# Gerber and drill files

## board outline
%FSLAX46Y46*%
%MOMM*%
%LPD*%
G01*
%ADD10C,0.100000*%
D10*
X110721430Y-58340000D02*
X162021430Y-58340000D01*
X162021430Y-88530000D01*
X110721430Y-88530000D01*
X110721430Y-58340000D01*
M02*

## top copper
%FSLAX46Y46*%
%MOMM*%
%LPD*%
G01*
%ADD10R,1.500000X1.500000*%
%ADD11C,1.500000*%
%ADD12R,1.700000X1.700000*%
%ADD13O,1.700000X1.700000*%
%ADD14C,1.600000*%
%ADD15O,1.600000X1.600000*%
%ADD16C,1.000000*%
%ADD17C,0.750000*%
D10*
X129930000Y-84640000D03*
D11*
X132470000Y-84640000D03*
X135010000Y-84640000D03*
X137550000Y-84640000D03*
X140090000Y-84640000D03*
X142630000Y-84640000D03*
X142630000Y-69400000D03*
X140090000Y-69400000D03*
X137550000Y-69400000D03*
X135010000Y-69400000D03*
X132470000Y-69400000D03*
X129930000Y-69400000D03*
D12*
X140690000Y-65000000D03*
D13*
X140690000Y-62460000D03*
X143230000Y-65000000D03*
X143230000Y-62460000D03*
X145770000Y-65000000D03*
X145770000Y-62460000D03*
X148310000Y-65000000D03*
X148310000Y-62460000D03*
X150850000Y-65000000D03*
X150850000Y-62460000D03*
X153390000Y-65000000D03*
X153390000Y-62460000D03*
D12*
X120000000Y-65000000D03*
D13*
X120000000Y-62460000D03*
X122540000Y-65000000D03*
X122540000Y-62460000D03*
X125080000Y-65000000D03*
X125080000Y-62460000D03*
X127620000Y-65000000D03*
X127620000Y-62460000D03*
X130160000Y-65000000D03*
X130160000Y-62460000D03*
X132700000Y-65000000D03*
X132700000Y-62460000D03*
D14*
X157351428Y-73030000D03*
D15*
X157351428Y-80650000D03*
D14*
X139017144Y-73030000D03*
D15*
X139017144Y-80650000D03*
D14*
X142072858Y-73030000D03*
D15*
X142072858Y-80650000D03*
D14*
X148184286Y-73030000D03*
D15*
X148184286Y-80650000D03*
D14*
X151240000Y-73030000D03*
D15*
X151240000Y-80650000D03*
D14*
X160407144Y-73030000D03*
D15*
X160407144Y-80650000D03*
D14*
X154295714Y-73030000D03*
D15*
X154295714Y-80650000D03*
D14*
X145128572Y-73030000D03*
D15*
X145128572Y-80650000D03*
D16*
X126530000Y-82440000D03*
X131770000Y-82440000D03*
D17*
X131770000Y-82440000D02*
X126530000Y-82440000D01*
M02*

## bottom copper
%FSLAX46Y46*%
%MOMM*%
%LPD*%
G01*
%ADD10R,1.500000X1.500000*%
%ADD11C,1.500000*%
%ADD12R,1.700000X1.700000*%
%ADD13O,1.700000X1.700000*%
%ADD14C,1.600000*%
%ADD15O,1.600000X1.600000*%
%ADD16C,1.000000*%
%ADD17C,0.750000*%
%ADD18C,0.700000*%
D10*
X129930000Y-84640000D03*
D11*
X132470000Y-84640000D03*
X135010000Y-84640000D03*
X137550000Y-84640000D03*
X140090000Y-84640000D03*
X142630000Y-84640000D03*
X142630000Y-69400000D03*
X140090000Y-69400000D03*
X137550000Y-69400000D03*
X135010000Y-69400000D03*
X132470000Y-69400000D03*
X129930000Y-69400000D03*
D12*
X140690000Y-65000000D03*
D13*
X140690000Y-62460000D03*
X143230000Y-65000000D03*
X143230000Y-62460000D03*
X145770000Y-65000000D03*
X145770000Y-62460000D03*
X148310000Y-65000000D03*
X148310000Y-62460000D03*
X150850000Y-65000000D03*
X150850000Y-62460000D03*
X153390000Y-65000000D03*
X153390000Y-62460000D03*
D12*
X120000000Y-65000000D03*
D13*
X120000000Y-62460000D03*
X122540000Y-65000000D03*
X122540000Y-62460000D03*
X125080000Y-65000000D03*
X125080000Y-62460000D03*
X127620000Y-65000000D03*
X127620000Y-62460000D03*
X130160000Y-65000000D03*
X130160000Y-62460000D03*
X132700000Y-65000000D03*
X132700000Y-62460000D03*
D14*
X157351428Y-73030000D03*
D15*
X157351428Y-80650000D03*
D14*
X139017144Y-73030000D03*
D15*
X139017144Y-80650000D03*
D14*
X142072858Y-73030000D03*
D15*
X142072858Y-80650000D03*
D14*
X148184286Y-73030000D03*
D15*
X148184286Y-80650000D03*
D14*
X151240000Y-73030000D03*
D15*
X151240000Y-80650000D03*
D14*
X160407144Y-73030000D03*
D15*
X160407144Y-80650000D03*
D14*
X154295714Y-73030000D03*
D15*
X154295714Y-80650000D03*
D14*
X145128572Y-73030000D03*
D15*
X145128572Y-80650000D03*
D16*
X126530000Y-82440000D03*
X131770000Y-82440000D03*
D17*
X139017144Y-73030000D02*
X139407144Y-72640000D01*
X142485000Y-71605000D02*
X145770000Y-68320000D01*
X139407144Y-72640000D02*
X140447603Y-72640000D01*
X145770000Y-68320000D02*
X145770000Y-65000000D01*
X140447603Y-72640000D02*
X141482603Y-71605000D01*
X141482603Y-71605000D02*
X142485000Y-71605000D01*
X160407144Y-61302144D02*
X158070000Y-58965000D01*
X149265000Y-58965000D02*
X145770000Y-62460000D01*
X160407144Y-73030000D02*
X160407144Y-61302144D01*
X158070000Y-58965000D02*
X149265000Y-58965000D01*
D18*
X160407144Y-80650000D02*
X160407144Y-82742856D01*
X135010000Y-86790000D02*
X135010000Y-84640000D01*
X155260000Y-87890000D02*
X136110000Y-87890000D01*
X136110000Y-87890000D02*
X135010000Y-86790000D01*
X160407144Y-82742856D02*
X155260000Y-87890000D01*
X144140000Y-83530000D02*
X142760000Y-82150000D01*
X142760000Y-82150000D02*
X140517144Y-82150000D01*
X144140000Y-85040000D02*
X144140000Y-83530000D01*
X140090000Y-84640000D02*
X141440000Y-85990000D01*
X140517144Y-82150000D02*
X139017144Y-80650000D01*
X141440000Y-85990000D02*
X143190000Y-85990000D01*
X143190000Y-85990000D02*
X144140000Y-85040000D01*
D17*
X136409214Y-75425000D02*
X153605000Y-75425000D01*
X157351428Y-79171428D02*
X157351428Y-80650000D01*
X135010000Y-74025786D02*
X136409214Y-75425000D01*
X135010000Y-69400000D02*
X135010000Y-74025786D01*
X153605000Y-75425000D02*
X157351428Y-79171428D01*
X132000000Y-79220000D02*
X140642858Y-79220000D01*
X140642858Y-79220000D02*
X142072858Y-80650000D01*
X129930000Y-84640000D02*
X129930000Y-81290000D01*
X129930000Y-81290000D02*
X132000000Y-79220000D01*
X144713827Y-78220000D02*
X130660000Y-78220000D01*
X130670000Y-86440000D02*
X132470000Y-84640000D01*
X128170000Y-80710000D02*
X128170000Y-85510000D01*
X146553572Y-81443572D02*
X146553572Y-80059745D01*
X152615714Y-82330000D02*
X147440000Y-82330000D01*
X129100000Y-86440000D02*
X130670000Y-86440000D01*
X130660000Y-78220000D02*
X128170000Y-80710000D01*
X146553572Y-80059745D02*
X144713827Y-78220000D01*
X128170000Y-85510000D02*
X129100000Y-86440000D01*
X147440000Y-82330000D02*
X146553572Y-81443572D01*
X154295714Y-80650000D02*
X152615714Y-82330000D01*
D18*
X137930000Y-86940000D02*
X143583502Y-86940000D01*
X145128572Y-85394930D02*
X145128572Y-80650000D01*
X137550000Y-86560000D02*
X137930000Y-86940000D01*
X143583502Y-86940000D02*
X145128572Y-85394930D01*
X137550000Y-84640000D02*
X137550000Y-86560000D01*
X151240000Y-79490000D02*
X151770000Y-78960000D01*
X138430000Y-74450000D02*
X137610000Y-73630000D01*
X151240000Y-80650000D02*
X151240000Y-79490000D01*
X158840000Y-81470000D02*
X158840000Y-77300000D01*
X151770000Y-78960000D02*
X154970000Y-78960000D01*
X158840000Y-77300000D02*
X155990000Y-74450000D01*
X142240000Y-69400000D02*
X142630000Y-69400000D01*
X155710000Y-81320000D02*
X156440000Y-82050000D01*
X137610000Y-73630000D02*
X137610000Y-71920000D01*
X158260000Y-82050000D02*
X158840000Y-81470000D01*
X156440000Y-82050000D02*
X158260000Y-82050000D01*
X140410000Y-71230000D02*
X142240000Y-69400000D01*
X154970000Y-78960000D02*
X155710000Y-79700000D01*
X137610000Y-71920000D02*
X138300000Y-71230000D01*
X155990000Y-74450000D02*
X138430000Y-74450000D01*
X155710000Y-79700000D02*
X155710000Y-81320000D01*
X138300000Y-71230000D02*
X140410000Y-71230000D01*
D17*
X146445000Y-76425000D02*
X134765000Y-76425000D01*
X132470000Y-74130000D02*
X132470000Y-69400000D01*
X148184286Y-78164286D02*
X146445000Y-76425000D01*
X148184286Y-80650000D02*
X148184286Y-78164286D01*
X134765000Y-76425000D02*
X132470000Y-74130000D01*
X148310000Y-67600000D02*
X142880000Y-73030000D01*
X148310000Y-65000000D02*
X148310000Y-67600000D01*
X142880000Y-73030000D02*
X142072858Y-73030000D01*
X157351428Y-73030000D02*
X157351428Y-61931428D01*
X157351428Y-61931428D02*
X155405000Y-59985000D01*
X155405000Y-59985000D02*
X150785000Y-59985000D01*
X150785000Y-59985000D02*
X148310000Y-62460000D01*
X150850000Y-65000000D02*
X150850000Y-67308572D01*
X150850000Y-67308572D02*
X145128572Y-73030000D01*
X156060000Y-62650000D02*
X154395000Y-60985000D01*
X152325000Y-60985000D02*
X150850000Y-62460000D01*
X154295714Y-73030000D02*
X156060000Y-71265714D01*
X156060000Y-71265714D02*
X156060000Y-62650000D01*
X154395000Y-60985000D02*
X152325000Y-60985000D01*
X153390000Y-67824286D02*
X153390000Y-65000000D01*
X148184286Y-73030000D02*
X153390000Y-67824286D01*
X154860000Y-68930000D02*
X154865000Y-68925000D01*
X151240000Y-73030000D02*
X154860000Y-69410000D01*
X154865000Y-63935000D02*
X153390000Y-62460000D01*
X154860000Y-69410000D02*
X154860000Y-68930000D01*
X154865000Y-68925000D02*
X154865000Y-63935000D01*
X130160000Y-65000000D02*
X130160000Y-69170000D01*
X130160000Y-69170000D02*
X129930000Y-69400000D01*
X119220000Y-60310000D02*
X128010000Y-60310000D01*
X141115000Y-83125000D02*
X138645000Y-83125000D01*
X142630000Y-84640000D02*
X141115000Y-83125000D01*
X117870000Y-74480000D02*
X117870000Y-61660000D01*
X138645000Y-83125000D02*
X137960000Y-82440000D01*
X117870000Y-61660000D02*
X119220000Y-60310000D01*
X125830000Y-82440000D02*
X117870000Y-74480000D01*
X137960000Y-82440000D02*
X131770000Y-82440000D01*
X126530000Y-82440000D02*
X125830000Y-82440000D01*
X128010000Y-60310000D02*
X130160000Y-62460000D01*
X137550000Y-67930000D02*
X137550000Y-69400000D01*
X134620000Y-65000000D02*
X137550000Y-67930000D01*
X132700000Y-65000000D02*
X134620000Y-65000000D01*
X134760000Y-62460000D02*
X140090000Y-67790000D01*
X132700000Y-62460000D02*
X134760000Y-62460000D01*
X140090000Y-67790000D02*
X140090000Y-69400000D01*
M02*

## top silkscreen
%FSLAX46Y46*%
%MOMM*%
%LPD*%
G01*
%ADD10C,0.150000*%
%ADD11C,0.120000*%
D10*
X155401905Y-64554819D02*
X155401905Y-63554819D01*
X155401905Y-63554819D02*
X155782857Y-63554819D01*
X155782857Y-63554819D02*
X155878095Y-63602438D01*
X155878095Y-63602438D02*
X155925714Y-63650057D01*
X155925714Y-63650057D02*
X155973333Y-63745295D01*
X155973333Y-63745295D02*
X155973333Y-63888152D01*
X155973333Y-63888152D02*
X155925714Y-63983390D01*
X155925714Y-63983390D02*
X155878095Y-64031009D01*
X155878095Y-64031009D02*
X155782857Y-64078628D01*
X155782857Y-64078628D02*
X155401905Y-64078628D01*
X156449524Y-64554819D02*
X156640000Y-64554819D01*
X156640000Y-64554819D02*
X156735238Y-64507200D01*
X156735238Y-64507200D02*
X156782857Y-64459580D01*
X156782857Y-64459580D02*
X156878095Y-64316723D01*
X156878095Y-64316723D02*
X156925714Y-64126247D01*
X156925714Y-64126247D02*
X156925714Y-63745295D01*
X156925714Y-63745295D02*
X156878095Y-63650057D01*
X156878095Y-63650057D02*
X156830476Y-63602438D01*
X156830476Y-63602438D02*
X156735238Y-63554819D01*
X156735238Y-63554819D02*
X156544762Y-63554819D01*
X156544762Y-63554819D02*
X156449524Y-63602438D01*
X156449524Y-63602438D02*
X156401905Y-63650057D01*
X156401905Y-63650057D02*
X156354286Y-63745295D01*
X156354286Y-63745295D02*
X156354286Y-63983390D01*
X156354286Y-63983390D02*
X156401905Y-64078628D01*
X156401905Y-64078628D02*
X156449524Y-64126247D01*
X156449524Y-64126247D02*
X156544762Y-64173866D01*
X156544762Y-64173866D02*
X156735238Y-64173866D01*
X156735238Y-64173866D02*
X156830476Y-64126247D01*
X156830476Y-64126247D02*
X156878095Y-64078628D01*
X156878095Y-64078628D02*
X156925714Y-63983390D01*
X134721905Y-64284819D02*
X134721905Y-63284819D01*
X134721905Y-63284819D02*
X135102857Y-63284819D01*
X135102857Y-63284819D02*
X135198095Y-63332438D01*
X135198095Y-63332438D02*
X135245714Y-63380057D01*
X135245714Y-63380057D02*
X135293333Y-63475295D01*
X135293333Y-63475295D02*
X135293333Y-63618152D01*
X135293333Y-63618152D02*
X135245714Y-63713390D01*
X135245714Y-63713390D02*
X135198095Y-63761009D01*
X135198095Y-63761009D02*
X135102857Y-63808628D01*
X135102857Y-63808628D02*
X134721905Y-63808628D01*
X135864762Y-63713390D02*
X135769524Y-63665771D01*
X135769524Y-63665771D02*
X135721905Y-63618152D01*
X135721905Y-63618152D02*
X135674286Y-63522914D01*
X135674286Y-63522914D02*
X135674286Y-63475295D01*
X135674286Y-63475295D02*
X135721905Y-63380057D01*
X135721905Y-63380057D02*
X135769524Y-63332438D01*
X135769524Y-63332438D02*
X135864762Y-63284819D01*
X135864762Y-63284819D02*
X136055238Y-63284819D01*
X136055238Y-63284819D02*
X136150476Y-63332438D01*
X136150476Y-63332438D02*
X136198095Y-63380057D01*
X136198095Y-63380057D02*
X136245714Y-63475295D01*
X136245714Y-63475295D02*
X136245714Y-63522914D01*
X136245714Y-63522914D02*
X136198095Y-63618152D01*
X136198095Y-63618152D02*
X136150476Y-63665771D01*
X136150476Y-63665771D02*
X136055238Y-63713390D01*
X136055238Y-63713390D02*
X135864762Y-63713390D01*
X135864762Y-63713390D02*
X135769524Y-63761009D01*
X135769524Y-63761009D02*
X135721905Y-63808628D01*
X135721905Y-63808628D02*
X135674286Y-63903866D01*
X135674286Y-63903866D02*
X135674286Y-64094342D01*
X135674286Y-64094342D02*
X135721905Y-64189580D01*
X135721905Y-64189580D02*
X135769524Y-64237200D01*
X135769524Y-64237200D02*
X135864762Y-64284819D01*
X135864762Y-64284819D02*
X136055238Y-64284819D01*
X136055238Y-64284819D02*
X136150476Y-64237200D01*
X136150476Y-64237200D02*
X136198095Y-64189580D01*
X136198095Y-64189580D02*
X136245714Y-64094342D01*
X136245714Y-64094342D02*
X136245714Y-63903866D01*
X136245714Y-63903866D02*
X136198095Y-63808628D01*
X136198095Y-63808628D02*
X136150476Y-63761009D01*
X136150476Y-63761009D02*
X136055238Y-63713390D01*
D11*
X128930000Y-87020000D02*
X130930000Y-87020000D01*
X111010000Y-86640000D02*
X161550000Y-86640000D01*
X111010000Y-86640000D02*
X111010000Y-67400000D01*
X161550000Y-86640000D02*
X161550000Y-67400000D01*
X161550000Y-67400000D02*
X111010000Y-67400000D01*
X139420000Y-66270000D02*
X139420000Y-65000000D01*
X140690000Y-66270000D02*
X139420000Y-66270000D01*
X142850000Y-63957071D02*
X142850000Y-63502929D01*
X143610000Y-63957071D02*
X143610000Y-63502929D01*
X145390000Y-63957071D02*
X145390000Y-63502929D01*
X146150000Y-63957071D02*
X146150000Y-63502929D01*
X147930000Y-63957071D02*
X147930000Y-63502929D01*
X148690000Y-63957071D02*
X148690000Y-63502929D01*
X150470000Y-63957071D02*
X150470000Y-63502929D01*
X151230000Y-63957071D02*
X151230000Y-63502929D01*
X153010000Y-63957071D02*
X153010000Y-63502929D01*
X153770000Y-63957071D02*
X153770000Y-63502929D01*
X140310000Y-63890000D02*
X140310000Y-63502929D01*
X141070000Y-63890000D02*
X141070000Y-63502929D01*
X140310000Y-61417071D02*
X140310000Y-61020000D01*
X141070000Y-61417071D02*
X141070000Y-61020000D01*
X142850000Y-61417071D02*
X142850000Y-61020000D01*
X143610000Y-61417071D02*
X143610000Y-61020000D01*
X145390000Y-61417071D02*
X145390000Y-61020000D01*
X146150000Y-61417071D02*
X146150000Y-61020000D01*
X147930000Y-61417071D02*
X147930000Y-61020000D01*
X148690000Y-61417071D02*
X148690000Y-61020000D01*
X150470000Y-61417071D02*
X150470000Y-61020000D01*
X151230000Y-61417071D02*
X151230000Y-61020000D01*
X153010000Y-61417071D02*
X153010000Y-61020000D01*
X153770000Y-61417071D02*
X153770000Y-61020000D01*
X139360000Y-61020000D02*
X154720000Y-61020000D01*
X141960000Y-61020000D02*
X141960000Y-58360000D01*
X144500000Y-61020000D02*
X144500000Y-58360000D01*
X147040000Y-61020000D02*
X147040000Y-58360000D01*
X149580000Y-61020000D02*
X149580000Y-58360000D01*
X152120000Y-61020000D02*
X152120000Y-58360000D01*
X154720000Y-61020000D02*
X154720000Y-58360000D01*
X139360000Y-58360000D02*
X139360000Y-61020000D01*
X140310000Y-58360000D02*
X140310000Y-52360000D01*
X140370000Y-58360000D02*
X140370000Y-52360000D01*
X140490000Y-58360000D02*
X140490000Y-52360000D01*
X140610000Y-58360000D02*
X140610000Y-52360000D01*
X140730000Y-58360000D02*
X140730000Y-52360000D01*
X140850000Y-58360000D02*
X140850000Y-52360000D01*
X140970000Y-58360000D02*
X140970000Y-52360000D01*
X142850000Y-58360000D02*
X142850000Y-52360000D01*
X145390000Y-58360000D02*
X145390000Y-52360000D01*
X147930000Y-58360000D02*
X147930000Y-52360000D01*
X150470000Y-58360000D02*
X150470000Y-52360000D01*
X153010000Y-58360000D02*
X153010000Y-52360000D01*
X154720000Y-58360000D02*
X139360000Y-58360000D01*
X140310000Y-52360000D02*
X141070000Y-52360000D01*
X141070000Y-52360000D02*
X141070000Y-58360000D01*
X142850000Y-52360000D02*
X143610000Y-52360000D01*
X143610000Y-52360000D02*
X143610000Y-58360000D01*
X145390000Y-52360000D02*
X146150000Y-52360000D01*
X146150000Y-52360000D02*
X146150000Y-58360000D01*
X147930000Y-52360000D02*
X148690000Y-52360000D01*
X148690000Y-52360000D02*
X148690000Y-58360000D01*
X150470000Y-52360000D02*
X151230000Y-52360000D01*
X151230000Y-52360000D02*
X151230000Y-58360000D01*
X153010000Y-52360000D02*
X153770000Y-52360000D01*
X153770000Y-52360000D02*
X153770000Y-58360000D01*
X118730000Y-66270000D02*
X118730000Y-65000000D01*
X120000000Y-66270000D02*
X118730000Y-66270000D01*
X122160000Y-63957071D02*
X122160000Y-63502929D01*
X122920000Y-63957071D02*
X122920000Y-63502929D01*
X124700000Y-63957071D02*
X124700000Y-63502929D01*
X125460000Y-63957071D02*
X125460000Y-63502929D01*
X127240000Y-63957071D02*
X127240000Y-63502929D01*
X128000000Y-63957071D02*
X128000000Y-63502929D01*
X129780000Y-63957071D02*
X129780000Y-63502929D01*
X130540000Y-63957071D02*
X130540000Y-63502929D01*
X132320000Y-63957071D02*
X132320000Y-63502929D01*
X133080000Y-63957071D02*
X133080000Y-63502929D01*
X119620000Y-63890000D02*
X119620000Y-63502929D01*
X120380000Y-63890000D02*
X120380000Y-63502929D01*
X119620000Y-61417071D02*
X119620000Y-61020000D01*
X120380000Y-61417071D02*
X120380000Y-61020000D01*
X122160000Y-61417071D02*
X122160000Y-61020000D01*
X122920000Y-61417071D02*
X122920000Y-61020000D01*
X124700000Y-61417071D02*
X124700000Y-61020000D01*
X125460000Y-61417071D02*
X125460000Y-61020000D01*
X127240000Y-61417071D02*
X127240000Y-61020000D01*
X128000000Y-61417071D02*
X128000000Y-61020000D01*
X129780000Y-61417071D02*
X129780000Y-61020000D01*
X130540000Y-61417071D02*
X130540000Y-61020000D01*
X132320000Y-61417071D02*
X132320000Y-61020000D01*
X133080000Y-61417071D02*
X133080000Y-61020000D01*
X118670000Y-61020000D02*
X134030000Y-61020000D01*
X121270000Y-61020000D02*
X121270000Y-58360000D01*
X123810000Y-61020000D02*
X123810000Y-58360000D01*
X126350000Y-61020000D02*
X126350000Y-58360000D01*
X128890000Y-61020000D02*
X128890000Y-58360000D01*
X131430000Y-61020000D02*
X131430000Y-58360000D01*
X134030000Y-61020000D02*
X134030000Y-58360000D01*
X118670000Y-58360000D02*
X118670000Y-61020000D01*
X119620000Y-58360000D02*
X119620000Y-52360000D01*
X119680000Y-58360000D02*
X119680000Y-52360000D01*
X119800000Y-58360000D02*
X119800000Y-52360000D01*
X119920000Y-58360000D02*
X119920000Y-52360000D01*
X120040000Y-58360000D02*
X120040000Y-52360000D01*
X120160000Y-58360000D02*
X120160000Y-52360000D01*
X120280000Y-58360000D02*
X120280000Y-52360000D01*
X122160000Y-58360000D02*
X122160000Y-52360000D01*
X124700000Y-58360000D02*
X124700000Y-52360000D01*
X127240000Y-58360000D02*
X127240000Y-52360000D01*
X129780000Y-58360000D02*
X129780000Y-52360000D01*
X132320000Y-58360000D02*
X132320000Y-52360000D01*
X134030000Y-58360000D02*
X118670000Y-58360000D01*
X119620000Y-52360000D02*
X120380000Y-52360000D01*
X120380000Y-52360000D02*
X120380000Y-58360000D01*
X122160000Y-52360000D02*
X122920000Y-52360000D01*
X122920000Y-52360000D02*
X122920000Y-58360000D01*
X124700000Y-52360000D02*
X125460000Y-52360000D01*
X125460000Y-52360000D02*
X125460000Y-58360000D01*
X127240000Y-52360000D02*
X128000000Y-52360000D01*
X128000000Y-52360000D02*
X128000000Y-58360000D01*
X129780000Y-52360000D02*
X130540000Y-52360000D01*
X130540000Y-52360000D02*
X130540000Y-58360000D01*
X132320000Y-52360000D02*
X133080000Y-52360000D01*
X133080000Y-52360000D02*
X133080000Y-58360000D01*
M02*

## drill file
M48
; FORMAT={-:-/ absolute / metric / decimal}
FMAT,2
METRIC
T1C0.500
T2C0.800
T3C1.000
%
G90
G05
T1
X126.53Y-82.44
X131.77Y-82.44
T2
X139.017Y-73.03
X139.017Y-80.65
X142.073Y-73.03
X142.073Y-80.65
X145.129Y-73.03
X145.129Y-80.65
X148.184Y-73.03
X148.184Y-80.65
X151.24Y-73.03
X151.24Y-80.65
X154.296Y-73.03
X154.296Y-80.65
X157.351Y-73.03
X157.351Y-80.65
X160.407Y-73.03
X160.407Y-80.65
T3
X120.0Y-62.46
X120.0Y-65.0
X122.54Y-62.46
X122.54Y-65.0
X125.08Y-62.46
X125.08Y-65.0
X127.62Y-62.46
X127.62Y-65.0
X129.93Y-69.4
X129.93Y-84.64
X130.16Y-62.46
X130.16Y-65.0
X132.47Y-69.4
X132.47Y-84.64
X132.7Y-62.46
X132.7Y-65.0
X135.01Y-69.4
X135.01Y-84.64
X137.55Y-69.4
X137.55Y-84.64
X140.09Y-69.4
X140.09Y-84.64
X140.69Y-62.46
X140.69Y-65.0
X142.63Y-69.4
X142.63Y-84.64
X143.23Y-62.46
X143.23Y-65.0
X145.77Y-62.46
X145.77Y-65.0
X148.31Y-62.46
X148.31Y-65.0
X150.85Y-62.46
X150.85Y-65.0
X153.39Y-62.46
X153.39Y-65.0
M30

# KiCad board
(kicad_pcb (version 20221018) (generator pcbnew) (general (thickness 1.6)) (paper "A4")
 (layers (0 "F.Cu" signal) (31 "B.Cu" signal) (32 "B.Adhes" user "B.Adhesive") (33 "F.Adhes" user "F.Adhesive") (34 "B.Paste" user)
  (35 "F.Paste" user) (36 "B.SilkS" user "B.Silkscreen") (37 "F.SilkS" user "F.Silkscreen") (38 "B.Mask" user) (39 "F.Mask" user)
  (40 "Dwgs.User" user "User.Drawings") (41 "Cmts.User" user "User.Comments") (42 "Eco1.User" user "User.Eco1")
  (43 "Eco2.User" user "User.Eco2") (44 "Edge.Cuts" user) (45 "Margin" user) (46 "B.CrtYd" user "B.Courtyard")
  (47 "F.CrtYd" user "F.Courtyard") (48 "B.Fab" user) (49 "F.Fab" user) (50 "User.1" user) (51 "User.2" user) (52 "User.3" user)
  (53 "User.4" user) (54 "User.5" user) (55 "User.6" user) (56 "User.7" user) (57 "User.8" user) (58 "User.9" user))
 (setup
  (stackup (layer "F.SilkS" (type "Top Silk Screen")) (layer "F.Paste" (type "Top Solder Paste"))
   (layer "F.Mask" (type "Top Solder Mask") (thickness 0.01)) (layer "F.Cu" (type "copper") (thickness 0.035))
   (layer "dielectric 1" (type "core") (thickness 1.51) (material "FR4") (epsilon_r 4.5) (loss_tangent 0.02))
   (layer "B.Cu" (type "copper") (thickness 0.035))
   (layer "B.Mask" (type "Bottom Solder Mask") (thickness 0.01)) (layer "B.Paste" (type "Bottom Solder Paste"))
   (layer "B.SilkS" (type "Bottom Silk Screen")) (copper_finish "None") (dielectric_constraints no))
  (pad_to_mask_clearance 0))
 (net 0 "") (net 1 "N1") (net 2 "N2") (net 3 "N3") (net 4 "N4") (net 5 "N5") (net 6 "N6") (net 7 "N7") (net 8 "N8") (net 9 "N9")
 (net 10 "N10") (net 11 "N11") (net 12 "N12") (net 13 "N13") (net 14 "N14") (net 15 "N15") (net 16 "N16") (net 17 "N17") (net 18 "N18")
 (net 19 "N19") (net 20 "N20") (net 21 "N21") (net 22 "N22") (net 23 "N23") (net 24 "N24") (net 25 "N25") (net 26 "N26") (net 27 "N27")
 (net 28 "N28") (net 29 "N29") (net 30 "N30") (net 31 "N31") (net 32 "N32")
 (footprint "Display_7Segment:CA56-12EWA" (layer "F.Cu") (at 129.93 84.64 90)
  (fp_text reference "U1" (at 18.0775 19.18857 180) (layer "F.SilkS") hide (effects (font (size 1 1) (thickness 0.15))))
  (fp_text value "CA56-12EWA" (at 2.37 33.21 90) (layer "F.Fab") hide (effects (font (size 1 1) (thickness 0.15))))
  (fp_line (start -2.38 -1) (end -2.38 1) (stroke (width 0.12) (type solid)) (layer "F.SilkS"))
  (fp_line (start -2 -18.92) (end -2 31.62) (stroke (width 0.12) (type solid)) (layer "F.SilkS"))
  (fp_line (start -2 -18.92) (end 17.24 -18.92) (stroke (width 0.12) (type solid)) (layer "F.SilkS"))
  (fp_line (start -2 31.62) (end 17.24 31.62) (stroke (width 0.12) (type solid)) (layer "F.SilkS"))
  (fp_line (start 17.24 31.62) (end 17.24 -18.92) (stroke (width 0.12) (type solid)) (layer "F.SilkS"))
  (pad "1" thru_hole rect (at 0 0 90) (size 1.5 1.5) (drill 1) (layers "*.Cu" "*.Mask") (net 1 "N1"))
  (pad "2" thru_hole circle (at 0 2.54 90) (size 1.5 1.5) (drill 1) (layers "*.Cu" "*.Mask") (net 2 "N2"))
  (pad "3" thru_hole circle (at 0 5.08 90) (size 1.5 1.5) (drill 1) (layers "*.Cu" "*.Mask") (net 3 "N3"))
  (pad "4" thru_hole circle (at 0 7.62 90) (size 1.5 1.5) (drill 1) (layers "*.Cu" "*.Mask") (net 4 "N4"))
  (pad "5" thru_hole circle (at 0 10.16 90) (size 1.5 1.5) (drill 1) (layers "*.Cu" "*.Mask") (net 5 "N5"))
  (pad "6" thru_hole circle (at 0 12.7 90) (size 1.5 1.5) (drill 1) (layers "*.Cu" "*.Mask") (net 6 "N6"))
  (pad "7" thru_hole circle (at 15.24 12.7 90) (size 1.5 1.5) (drill 1) (layers "*.Cu" "*.Mask") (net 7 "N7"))
  (pad "8" thru_hole circle (at 15.24 10.16 90) (size 1.5 1.5) (drill 1) (layers "*.Cu" "*.Mask") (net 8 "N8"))
  (pad "9" thru_hole circle (at 15.24 7.62 90) (size 1.5 1.5) (drill 1) (layers "*.Cu" "*.Mask") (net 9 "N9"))
  (pad "10" thru_hole circle (at 15.24 5.08 90) (size 1.5 1.5) (drill 1) (layers "*.Cu" "*.Mask") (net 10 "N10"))
  (pad "11" thru_hole circle (at 15.24 2.54 90) (size 1.5 1.5) (drill 1) (layers "*.Cu" "*.Mask") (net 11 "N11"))
  (pad "12" thru_hole circle (at 15.24 0 90) (size 1.5 1.5) (drill 1) (layers "*.Cu" "*.Mask") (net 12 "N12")))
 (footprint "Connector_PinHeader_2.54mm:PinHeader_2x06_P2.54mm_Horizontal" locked (layer "F.Cu") (at 140.69 65 90)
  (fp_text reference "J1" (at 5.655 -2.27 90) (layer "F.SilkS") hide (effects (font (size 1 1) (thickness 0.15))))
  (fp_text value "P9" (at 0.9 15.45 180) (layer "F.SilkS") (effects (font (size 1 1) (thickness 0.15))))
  (fp_line (start -1.27 -1.27) (end 0 -1.27) (stroke (width 0.12) (type solid)) (layer "F.SilkS"))
  (fp_line (start -1.27 0) (end -1.27 -1.27) (stroke (width 0.12) (type solid)) (layer "F.SilkS"))
  (fp_line (start 1.042929 2.16) (end 1.497071 2.16) (stroke (width 0.12) (type solid)) (layer "F.SilkS"))
  (fp_line (start 1.042929 2.92) (end 1.497071 2.92) (stroke (width 0.12) (type solid)) (layer "F.SilkS"))
  (fp_line (start 1.042929 4.7) (end 1.497071 4.7) (stroke (width 0.12) (type solid)) (layer "F.SilkS"))
  (fp_line (start 1.042929 5.46) (end 1.497071 5.46) (stroke (width 0.12) (type solid)) (layer "F.SilkS"))
  (fp_line (start 1.042929 7.24) (end 1.497071 7.24) (stroke (width 0.12) (type solid)) (layer "F.SilkS"))
  (fp_line (start 1.042929 8) (end 1.497071 8) (stroke (width 0.12) (type solid)) (layer "F.SilkS"))
  (fp_line (start 1.042929 9.78) (end 1.497071 9.78) (stroke (width 0.12) (type solid)) (layer "F.SilkS"))
  (fp_line (start 1.042929 10.54) (end 1.497071 10.54) (stroke (width 0.12) (type solid)) (layer "F.SilkS"))
  (fp_line (start 1.042929 12.32) (end 1.497071 12.32) (stroke (width 0.12) (type solid)) (layer "F.SilkS"))
  (fp_line (start 1.042929 13.08) (end 1.497071 13.08) (stroke (width 0.12) (type solid)) (layer "F.SilkS"))
  (fp_line (start 1.11 -0.38) (end 1.497071 -0.38) (stroke (width 0.12) (type solid)) (layer "F.SilkS"))
  (fp_line (start 1.11 0.38) (end 1.497071 0.38) (stroke (width 0.12) (type solid)) (layer "F.SilkS"))
  (fp_line (start 3.582929 -0.38) (end 3.98 -0.38) (stroke (width 0.12) (type solid)) (layer "F.SilkS"))
  (fp_line (start 3.582929 0.38) (end 3.98 0.38) (stroke (width 0.12) (type solid)) (layer "F.SilkS"))
  (fp_line (start 3.582929 2.16) (end 3.98 2.16) (stroke (width 0.12) (type solid)) (layer "F.SilkS"))
  (fp_line (start 3.582929 2.92) (end 3.98 2.92) (stroke (width 0.12) (type solid)) (layer "F.SilkS"))
  (fp_line (start 3.582929 4.7) (end 3.98 4.7) (stroke (width 0.12) (type solid)) (layer "F.SilkS"))
  (fp_line (start 3.582929 5.46) (end 3.98 5.46) (stroke (width 0.12) (type solid)) (layer "F.SilkS"))
  (fp_line (start 3.582929 7.24) (end 3.98 7.24) (stroke (width 0.12) (type solid)) (layer "F.SilkS"))
  (fp_line (start 3.582929 8) (end 3.98 8) (stroke (width 0.12) (type solid)) (layer "F.SilkS"))
  (fp_line (start 3.582929 9.78) (end 3.98 9.78) (stroke (width 0.12) (type solid)) (layer "F.SilkS"))
  (fp_line (start 3.582929 10.54) (end 3.98 10.54) (stroke (width 0.12) (type solid)) (layer "F.SilkS"))
  (fp_line (start 3.582929 12.32) (end 3.98 12.32) (stroke (width 0.12) (type solid)) (layer "F.SilkS"))
  (fp_line (start 3.582929 13.08) (end 3.98 13.08) (stroke (width 0.12) (type solid)) (layer "F.SilkS"))
  (fp_line (start 3.98 -1.33) (end 3.98 14.03) (stroke (width 0.12) (type solid)) (layer "F.SilkS"))
  (fp_line (start 3.98 1.27) (end 6.64 1.27) (stroke (width 0.12) (type solid)) (layer "F.SilkS"))
  (fp_line (start 3.98 3.81) (end 6.64 3.81) (stroke (width 0.12) (type solid)) (layer "F.SilkS"))
  (fp_line (start 3.98 6.35) (end 6.64 6.35) (stroke (width 0.12) (type solid)) (layer "F.SilkS"))
  (fp_line (start 3.98 8.89) (end 6.64 8.89) (stroke (width 0.12) (type solid)) (layer "F.SilkS"))
  (fp_line (start 3.98 11.43) (end 6.64 11.43) (stroke (width 0.12) (type solid)) (layer "F.SilkS"))
  (fp_line (start 3.98 14.03) (end 6.64 14.03) (stroke (width 0.12) (type solid)) (layer "F.SilkS"))
  (fp_line (start 6.64 -1.33) (end 3.98 -1.33) (stroke (width 0.12) (type solid)) (layer "F.SilkS"))
  (fp_line (start 6.64 -0.38) (end 12.64 -0.38) (stroke (width 0.12) (type solid)) (layer "F.SilkS"))
  (fp_line (start 6.64 -0.32) (end 12.64 -0.32) (stroke (width 0.12) (type solid)) (layer "F.SilkS"))
  (fp_line (start 6.64 -0.2) (end 12.64 -0.2) (stroke (width 0.12) (type solid)) (layer "F.SilkS"))
  (fp_line (start 6.64 -0.08) (end 12.64 -0.08) (stroke (width 0.12) (type solid)) (layer "F.SilkS"))
  (fp_line (start 6.64 0.04) (end 12.64 0.04) (stroke (width 0.12) (type solid)) (layer "F.SilkS"))
  (fp_line (start 6.64 0.16) (end 12.64 0.16) (stroke (width 0.12) (type solid)) (layer "F.SilkS"))
  (fp_line (start 6.64 0.28) (end 12.64 0.28) (stroke (width 0.12) (type solid)) (layer "F.SilkS"))
  (fp_line (start 6.64 2.16) (end 12.64 2.16) (stroke (width 0.12) (type solid)) (layer "F.SilkS"))
  (fp_line (start 6.64 4.7) (end 12.64 4.7) (stroke (width 0.12) (type solid)) (layer "F.SilkS"))
  (fp_line (start 6.64 7.24) (end 12.64 7.24) (stroke (width 0.12) (type solid)) (layer "F.SilkS"))
  (fp_line (start 6.64 9.78) (end 12.64 9.78) (stroke (width 0.12) (type solid)) (layer "F.SilkS"))
  (fp_line (start 6.64 12.32) (end 12.64 12.32) (stroke (width 0.12) (type solid)) (layer "F.SilkS"))
  (fp_line (start 6.64 14.03) (end 6.64 -1.33) (stroke (width 0.12) (type solid)) (layer "F.SilkS"))
  (fp_line (start 12.64 -0.38) (end 12.64 0.38) (stroke (width 0.12) (type solid)) (layer "F.SilkS"))
  (fp_line (start 12.64 0.38) (end 6.64 0.38) (stroke (width 0.12) (type solid)) (layer "F.SilkS"))
  (fp_line (start 12.64 2.16) (end 12.64 2.92) (stroke (width 0.12) (type solid)) (layer "F.SilkS"))
  (fp_line (start 12.64 2.92) (end 6.64 2.92) (stroke (width 0.12) (type solid)) (layer "F.SilkS"))
  (fp_line (start 12.64 4.7) (end 12.64 5.46) (stroke (width 0.12) (type solid)) (layer "F.SilkS"))
  (fp_line (start 12.64 5.46) (end 6.64 5.46) (stroke (width 0.12) (type solid)) (layer "F.SilkS"))
  (fp_line (start 12.64 7.24) (end 12.64 8) (stroke (width 0.12) (type solid)) (layer "F.SilkS"))
  (fp_line (start 12.64 8) (end 6.64 8) (stroke (width 0.12) (type solid)) (layer "F.SilkS"))
  (fp_line (start 12.64 9.78) (end 12.64 10.54) (stroke (width 0.12) (type solid)) (layer "F.SilkS"))
  (fp_line (start 12.64 10.54) (end 6.64 10.54) (stroke (width 0.12) (type solid)) (layer "F.SilkS"))
  (fp_line (start 12.64 12.32) (end 12.64 13.08) (stroke (width 0.12) (type solid)) (layer "F.SilkS"))
  (fp_line (start 12.64 13.08) (end 6.64 13.08) (stroke (width 0.12) (type solid)) (layer "F.SilkS"))
  (pad "1" thru_hole rect locked (at 0 0 90) (size 1.7 1.7) (drill 1) (layers "*.Cu" "*.Mask") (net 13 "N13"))
  (pad "2" thru_hole oval locked (at 2.54 0 90) (size 1.7 1.7) (drill 1) (layers "*.Cu" "*.Mask") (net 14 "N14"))
  (pad "3" thru_hole oval locked (at 0 2.54 90) (size 1.7 1.7) (drill 1) (layers "*.Cu" "*.Mask") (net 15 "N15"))
  (pad "4" thru_hole oval locked (at 2.54 2.54 90) (size 1.7 1.7) (drill 1) (layers "*.Cu" "*.Mask") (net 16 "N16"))
  (pad "5" thru_hole oval locked (at 0 5.08 90) (size 1.7 1.7) (drill 1) (layers "*.Cu" "*.Mask") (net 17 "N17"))
  (pad "6" thru_hole oval locked (at 2.54 5.08 90) (size 1.7 1.7) (drill 1) (layers "*.Cu" "*.Mask") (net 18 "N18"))
  (pad "7" thru_hole oval locked (at 0 7.62 90) (size 1.7 1.7) (drill 1) (layers "*.Cu" "*.Mask") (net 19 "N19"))
  (pad "8" thru_hole oval locked (at 2.54 7.62 90) (size 1.7 1.7) (drill 1) (layers "*.Cu" "*.Mask") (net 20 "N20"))
  (pad "9" thru_hole oval locked (at 0 10.16 90) (size 1.7 1.7) (drill 1) (layers "*.Cu" "*.Mask") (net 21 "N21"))
  (pad "10" thru_hole oval locked (at 2.54 10.16 90) (size 1.7 1.7) (drill 1) (layers "*.Cu" "*.Mask") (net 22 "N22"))
  (pad "11" thru_hole oval locked (at 0 12.7 90) (size 1.7 1.7) (drill 1) (layers "*.Cu" "*.Mask") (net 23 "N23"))
  (pad "12" thru_hole oval locked (at 2.54 12.7 90) (size 1.7 1.7) (drill 1) (layers "*.Cu" "*.Mask") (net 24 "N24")))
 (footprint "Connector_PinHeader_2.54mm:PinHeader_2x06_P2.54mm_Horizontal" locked (layer "F.Cu") (at 120 65 90)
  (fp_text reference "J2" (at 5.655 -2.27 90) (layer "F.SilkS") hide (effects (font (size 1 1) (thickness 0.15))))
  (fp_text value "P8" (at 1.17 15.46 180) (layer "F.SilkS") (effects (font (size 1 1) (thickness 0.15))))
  (fp_line (start -1.27 -1.27) (end 0 -1.27) (stroke (width 0.12) (type solid)) (layer "F.SilkS"))
  (fp_line (start -1.27 0) (end -1.27 -1.27) (stroke (width 0.12) (type solid)) (layer "F.SilkS"))
  (fp_line (start 1.042929 2.16) (end 1.497071 2.16) (stroke (width 0.12) (type solid)) (layer "F.SilkS"))
  (fp_line (start 1.042929 2.92) (end 1.497071 2.92) (stroke (width 0.12) (type solid)) (layer "F.SilkS"))
  (fp_line (start 1.042929 4.7) (end 1.497071 4.7) (stroke (width 0.12) (type solid)) (layer "F.SilkS"))
  (fp_line (start 1.042929 5.46) (end 1.497071 5.46) (stroke (width 0.12) (type solid)) (layer "F.SilkS"))
  (fp_line (start 1.042929 7.24) (end 1.497071 7.24) (stroke (width 0.12) (type solid)) (layer "F.SilkS"))
  (fp_line (start 1.042929 8) (end 1.497071 8) (stroke (width 0.12) (type solid)) (layer "F.SilkS"))
  (fp_line (start 1.042929 9.78) (end 1.497071 9.78) (stroke (width 0.12) (type solid)) (layer "F.SilkS"))
  (fp_line (start 1.042929 10.54) (end 1.497071 10.54) (stroke (width 0.12) (type solid)) (layer "F.SilkS"))
  (fp_line (start 1.042929 12.32) (end 1.497071 12.32) (stroke (width 0.12) (type solid)) (layer "F.SilkS"))
  (fp_line (start 1.042929 13.08) (end 1.497071 13.08) (stroke (width 0.12) (type solid)) (layer "F.SilkS"))
  (fp_line (start 1.11 -0.38) (end 1.497071 -0.38) (stroke (width 0.12) (type solid)) (layer "F.SilkS"))
  (fp_line (start 1.11 0.38) (end 1.497071 0.38) (stroke (width 0.12) (type solid)) (layer "F.SilkS"))
  (fp_line (start 3.582929 -0.38) (end 3.98 -0.38) (stroke (width 0.12) (type solid)) (layer "F.SilkS"))
  (fp_line (start 3.582929 0.38) (end 3.98 0.38) (stroke (width 0.12) (type solid)) (layer "F.SilkS"))
  (fp_line (start 3.582929 2.16) (end 3.98 2.16) (stroke (width 0.12) (type solid)) (layer "F.SilkS"))
  (fp_line (start 3.582929 2.92) (end 3.98 2.92) (stroke (width 0.12) (type solid)) (layer "F.SilkS"))
  (fp_line (start 3.582929 4.7) (end 3.98 4.7) (stroke (width 0.12) (type solid)) (layer "F.SilkS"))
  (fp_line (start 3.582929 5.46) (end 3.98 5.46) (stroke (width 0.12) (type solid)) (layer "F.SilkS"))
  (fp_line (start 3.582929 7.24) (end 3.98 7.24) (stroke (width 0.12) (type solid)) (layer "F.SilkS"))
  (fp_line (start 3.582929 8) (end 3.98 8) (stroke (width 0.12) (type solid)) (layer "F.SilkS"))
  (fp_line (start 3.582929 9.78) (end 3.98 9.78) (stroke (width 0.12) (type solid)) (layer "F.SilkS"))
  (fp_line (start 3.582929 10.54) (end 3.98 10.54) (stroke (width 0.12) (type solid)) (layer "F.SilkS"))
  (fp_line (start 3.582929 12.32) (end 3.98 12.32) (stroke (width 0.12) (type solid)) (layer "F.SilkS"))
  (fp_line (start 3.582929 13.08) (end 3.98 13.08) (stroke (width 0.12) (type solid)) (layer "F.SilkS"))
  (fp_line (start 3.98 -1.33) (end 3.98 14.03) (stroke (width 0.12) (type solid)) (layer "F.SilkS"))
  (fp_line (start 3.98 1.27) (end 6.64 1.27) (stroke (width 0.12) (type solid)) (layer "F.SilkS"))
  (fp_line (start 3.98 3.81) (end 6.64 3.81) (stroke (width 0.12) (type solid)) (layer "F.SilkS"))
  (fp_line (start 3.98 6.35) (end 6.64 6.35) (stroke (width 0.12) (type solid)) (layer "F.SilkS"))
  (fp_line (start 3.98 8.89) (end 6.64 8.89) (stroke (width 0.12) (type solid)) (layer "F.SilkS"))
  (fp_line (start 3.98 11.43) (end 6.64 11.43) (stroke (width 0.12) (type solid)) (layer "F.SilkS"))
  (fp_line (start 3.98 14.03) (end 6.64 14.03) (stroke (width 0.12) (type solid)) (layer "F.SilkS"))
  (fp_line (start 6.64 -1.33) (end 3.98 -1.33) (stroke (width 0.12) (type solid)) (layer "F.SilkS"))
  (fp_line (start 6.64 -0.38) (end 12.64 -0.38) (stroke (width 0.12) (type solid)) (layer "F.SilkS"))
  (fp_line (start 6.64 -0.32) (end 12.64 -0.32) (stroke (width 0.12) (type solid)) (layer "F.SilkS"))
  (fp_line (start 6.64 -0.2) (end 12.64 -0.2) (stroke (width 0.12) (type solid)) (layer "F.SilkS"))
  (fp_line (start 6.64 -0.08) (end 12.64 -0.08) (stroke (width 0.12) (type solid)) (layer "F.SilkS"))
  (fp_line (start 6.64 0.04) (end 12.64 0.04) (stroke (width 0.12) (type solid)) (layer "F.SilkS"))
  (fp_line (start 6.64 0.16) (end 12.64 0.16) (stroke (width 0.12) (type solid)) (layer "F.SilkS"))
  (fp_line (start 6.64 0.28) (end 12.64 0.28) (stroke (width 0.12) (type solid)) (layer "F.SilkS"))
  (fp_line (start 6.64 2.16) (end 12.64 2.16) (stroke (width 0.12) (type solid)) (layer "F.SilkS"))
  (fp_line (start 6.64 4.7) (end 12.64 4.7) (stroke (width 0.12) (type solid)) (layer "F.SilkS"))
  (fp_line (start 6.64 7.24) (end 12.64 7.24) (stroke (width 0.12) (type solid)) (layer "F.SilkS"))
  (fp_line (start 6.64 9.78) (end 12.64 9.78) (stroke (width 0.12) (type solid)) (layer "F.SilkS"))
  (fp_line (start 6.64 12.32) (end 12.64 12.32) (stroke (width 0.12) (type solid)) (layer "F.SilkS"))
  (fp_line (start 6.64 14.03) (end 6.64 -1.33) (stroke (width 0.12) (type solid)) (layer "F.SilkS"))
  (fp_line (start 12.64 -0.38) (end 12.64 0.38) (stroke (width 0.12) (type solid)) (layer "F.SilkS"))
  (fp_line (start 12.64 0.38) (end 6.64 0.38) (stroke (width 0.12) (type solid)) (layer "F.SilkS"))
  (fp_line (start 12.64 2.16) (end 12.64 2.92) (stroke (width 0.12) (type solid)) (layer "F.SilkS"))
  (fp_line (start 12.64 2.92) (end 6.64 2.92) (stroke (width 0.12) (type solid)) (layer "F.SilkS"))
  (fp_line (start 12.64 4.7) (end 12.64 5.46) (stroke (width 0.12) (type solid)) (layer "F.SilkS"))
  (fp_line (start 12.64 5.46) (end 6.64 5.46) (stroke (width 0.12) (type solid)) (layer "F.SilkS"))
  (fp_line (start 12.64 7.24) (end 12.64 8) (stroke (width 0.12) (type solid)) (layer "F.SilkS"))
  (fp_line (start 12.64 8) (end 6.64 8) (stroke (width 0.12) (type solid)) (layer "F.SilkS"))
  (fp_line (start 12.64 9.78) (end 12.64 10.54) (stroke (width 0.12) (type solid)) (layer "F.SilkS"))
  (fp_line (start 12.64 10.54) (end 6.64 10.54) (stroke (width 0.12) (type solid)) (layer "F.SilkS"))
  (fp_line (start 12.64 12.32) (end 12.64 13.08) (stroke (width 0.12) (type solid)) (layer "F.SilkS"))
  (fp_line (start 12.64 13.08) (end 6.64 13.08) (stroke (width 0.12) (type solid)) (layer "F.SilkS"))
  (pad "1" thru_hole rect locked (at 0 0 90) (size 1.7 1.7) (drill 1) (layers "*.Cu" "*.Mask") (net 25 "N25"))
  (pad "2" thru_hole oval locked (at 2.54 0 90) (size 1.7 1.7) (drill 1) (layers "*.Cu" "*.Mask") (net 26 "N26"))
  (pad "3" thru_hole oval locked (at 0 2.54 90) (size 1.7 1.7) (drill 1) (layers "*.Cu" "*.Mask") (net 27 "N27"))
  (pad "4" thru_hole oval locked (at 2.54 2.54 90) (size 1.7 1.7) (drill 1) (layers "*.Cu" "*.Mask") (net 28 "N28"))
  (pad "5" thru_hole oval locked (at 0 5.08 90) (size 1.7 1.7) (drill 1) (layers "*.Cu" "*.Mask") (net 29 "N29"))
  (pad "6" thru_hole oval locked (at 2.54 5.08 90) (size 1.7 1.7) (drill 1) (layers "*.Cu" "*.Mask") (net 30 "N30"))
  (pad "7" thru_hole oval locked (at 0 7.62 90) (size 1.7 1.7) (drill 1) (layers "*.Cu" "*.Mask") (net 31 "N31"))
  (pad "8" thru_hole oval locked (at 2.54 7.62 90) (size 1.7 1.7) (drill 1) (layers "*.Cu" "*.Mask") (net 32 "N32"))
  (pad "9" thru_hole oval locked (at 0 10.16 90) (size 1.7 1.7) (drill 1) (layers "*.Cu" "*.Mask") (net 12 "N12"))
  (pad "10" thru_hole oval locked (at 2.54 10.16 90) (size 1.7 1.7) (drill 1) (layers "*.Cu" "*.Mask") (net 6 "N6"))
  (pad "11" thru_hole oval locked (at 0 12.7 90) (size 1.7 1.7) (drill 1) (layers "*.Cu" "*.Mask") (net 9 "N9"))
  (pad "12" thru_hole oval locked (at 2.54 12.7 90) (size 1.7 1.7) (drill 1) (layers "*.Cu" "*.Mask") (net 8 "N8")))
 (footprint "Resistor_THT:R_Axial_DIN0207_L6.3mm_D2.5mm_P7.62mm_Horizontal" (layer "B.Cu") (at 157.351428 73.03 -90)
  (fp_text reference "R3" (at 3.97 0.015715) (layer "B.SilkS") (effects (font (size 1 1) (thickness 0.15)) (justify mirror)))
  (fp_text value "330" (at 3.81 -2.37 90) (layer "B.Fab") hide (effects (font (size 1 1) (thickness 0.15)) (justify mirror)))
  (pad "1" thru_hole circle (at 0 0 270) (size 1.6 1.6) (drill 0.8) (layers "*.Cu" "*.Mask") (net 20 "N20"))
  (pad "2" thru_hole oval (at 7.62 0 270) (size 1.6 1.6) (drill 0.8) (layers "*.Cu" "*.Mask") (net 10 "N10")))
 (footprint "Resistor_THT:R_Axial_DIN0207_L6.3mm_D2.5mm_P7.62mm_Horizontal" (layer "B.Cu") (at 139.017144 73.03 -90)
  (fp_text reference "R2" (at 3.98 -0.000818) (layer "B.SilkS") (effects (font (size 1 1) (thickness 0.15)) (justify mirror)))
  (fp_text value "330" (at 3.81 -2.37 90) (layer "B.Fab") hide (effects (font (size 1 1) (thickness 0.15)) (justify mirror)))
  (pad "1" thru_hole circle (at 0 0 270) (size 1.6 1.6) (drill 0.8) (layers "*.Cu" "*.Mask") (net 17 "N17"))
  (pad "2" thru_hole oval (at 7.62 0 270) (size 1.6 1.6) (drill 0.8) (layers "*.Cu" "*.Mask") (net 5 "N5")))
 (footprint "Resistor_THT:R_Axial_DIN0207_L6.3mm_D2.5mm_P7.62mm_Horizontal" (layer "B.Cu") (at 142.072858 73.03 -90)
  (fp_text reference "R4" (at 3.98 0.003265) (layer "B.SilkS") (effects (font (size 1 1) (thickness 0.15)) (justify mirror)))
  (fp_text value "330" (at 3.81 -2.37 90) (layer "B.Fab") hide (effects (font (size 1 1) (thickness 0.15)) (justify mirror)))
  (pad "1" thru_hole circle (at 0 0 270) (size 1.6 1.6) (drill 0.8) (layers "*.Cu" "*.Mask") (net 19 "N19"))
  (pad "2" thru_hole oval (at 7.62 0 270) (size 1.6 1.6) (drill 0.8) (layers "*.Cu" "*.Mask") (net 1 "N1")))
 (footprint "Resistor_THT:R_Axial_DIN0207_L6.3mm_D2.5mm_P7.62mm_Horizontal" (layer "B.Cu") (at 148.184286 73.03 -90)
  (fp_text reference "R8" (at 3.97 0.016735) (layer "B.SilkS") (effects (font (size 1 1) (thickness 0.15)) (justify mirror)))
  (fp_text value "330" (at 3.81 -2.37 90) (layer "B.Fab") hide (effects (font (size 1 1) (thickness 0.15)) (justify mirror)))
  (pad "1" thru_hole circle (at 0 0 270) (size 1.6 1.6) (drill 0.8) (layers "*.Cu" "*.Mask") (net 23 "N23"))
  (pad "2" thru_hole oval (at 7.62 0 270) (size 1.6 1.6) (drill 0.8) (layers "*.Cu" "*.Mask") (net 11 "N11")))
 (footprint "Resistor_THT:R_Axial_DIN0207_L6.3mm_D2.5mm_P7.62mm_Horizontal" (layer "B.Cu") (at 151.24 73.03 -90)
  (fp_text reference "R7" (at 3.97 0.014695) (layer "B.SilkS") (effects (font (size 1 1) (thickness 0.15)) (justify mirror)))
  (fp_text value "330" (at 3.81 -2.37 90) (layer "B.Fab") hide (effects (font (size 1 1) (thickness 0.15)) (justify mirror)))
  (pad "1" thru_hole circle (at 0 0 270) (size 1.6 1.6) (drill 0.8) (layers "*.Cu" "*.Mask") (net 24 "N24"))
  (pad "2" thru_hole oval (at 7.62 0 270) (size 1.6 1.6) (drill 0.8) (layers "*.Cu" "*.Mask") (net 7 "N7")))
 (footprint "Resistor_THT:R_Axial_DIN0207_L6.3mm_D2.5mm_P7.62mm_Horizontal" (layer "B.Cu") (at 160.407144 73.03 -90)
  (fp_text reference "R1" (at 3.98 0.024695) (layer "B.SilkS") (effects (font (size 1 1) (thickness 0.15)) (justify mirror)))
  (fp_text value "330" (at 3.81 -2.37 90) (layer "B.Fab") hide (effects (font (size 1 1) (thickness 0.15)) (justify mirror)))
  (pad "1" thru_hole circle (at 0 0 270) (size 1.6 1.6) (drill 0.8) (layers "*.Cu" "*.Mask") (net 18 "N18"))
  (pad "2" thru_hole oval (at 7.62 0 270) (size 1.6 1.6) (drill 0.8) (layers "*.Cu" "*.Mask") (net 3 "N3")))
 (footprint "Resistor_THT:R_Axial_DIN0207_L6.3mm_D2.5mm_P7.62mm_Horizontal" (layer "B.Cu") (at 154.295714 73.03 -90)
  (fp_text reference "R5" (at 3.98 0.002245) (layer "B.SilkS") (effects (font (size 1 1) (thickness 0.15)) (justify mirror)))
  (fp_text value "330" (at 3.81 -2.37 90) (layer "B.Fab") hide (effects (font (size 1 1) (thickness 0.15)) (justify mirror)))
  (pad "1" thru_hole circle (at 0 0 270) (size 1.6 1.6) (drill 0.8) (layers "*.Cu" "*.Mask") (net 22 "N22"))
  (pad "2" thru_hole oval (at 7.62 0 270) (size 1.6 1.6) (drill 0.8) (layers "*.Cu" "*.Mask") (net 2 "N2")))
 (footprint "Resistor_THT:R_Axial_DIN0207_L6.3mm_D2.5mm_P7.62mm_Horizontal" (layer "B.Cu") (at 145.128572 73.03 -90)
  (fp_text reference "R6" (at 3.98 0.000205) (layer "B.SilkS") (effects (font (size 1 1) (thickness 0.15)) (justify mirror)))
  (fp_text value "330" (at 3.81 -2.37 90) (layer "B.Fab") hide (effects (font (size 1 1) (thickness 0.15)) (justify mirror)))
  (pad "1" thru_hole circle (at 0 0 270) (size 1.6 1.6) (drill 0.8) (layers "*.Cu" "*.Mask") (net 21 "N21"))
  (pad "2" thru_hole oval (at 7.62 0 270) (size 1.6 1.6) (drill 0.8) (layers "*.Cu" "*.Mask") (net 4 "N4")))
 (gr_rect (start 110.72143 58.34) (end 162.02143 88.53) (stroke (width 0.1) (type solid)) (fill none) (layer "Edge.Cuts"))
 (segment (start 139.017144 73.03) (end 139.407144 72.64) (width 0.75) (layer "B.Cu") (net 17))
 (segment (start 142.485 71.605) (end 145.77 68.32) (width 0.75) (layer "B.Cu") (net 17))
 (segment (start 139.407144 72.64) (end 140.447603 72.64) (width 0.75) (layer "B.Cu") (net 17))
 (segment (start 145.77 68.32) (end 145.77 65) (width 0.75) (layer "B.Cu") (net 17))
 (segment (start 140.447603 72.64) (end 141.482603 71.605) (width 0.75) (layer "B.Cu") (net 17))
 (segment (start 141.482603 71.605) (end 142.485 71.605) (width 0.75) (layer "B.Cu") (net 17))
 (segment (start 160.407144 61.302144) (end 158.07 58.965) (width 0.75) (layer "B.Cu") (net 18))
 (segment (start 149.265 58.965) (end 145.77 62.46) (width 0.75) (layer "B.Cu") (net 18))
 (segment (start 160.407144 73.03) (end 160.407144 61.302144) (width 0.75) (layer "B.Cu") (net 18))
 (segment (start 158.07 58.965) (end 149.265 58.965) (width 0.75) (layer "B.Cu") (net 18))
 (segment (start 160.407144 80.65) (end 160.407144 82.742856) (width 0.7) (layer "B.Cu") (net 3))
 (segment (start 135.01 86.79) (end 135.01 84.64) (width 0.7) (layer "B.Cu") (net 3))
 (segment (start 155.26 87.89) (end 136.11 87.89) (width 0.7) (layer "B.Cu") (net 3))
 (segment (start 136.11 87.89) (end 135.01 86.79) (width 0.7) (layer "B.Cu") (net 3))
 (segment (start 160.407144 82.742856) (end 155.26 87.89) (width 0.7) (layer "B.Cu") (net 3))
 (segment (start 144.14 83.53) (end 142.76 82.15) (width 0.7) (layer "B.Cu") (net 5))
 (segment (start 142.76 82.15) (end 140.517144 82.15) (width 0.7) (layer "B.Cu") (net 5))
 (segment (start 144.14 85.04) (end 144.14 83.53) (width 0.7) (layer "B.Cu") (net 5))
 (segment (start 140.09 84.64) (end 141.44 85.99) (width 0.7) (layer "B.Cu") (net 5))
 (segment (start 140.517144 82.15) (end 139.017144 80.65) (width 0.7) (layer "B.Cu") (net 5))
 (segment (start 141.44 85.99) (end 143.19 85.99) (width 0.7) (layer "B.Cu") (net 5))
 (segment (start 143.19 85.99) (end 144.14 85.04) (width 0.7) (layer "B.Cu") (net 5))
 (segment (start 136.409214 75.425) (end 153.605 75.425) (width 0.75) (layer "B.Cu") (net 10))
 (segment (start 157.351428 79.171428) (end 157.351428 80.65) (width 0.75) (layer "B.Cu") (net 10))
 (segment (start 135.01 74.025786) (end 136.409214 75.425) (width 0.75) (layer "B.Cu") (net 10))
 (segment (start 135.01 69.4) (end 135.01 74.025786) (width 0.75) (layer "B.Cu") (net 10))
 (segment (start 153.605 75.425) (end 157.351428 79.171428) (width 0.75) (layer "B.Cu") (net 10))
 (segment (start 132 79.22) (end 140.642858 79.22) (width 0.75) (layer "B.Cu") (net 1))
 (segment (start 140.642858 79.22) (end 142.072858 80.65) (width 0.75) (layer "B.Cu") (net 1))
 (segment (start 129.93 84.64) (end 129.93 81.29) (width 0.75) (layer "B.Cu") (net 1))
 (segment (start 129.93 81.29) (end 132 79.22) (width 0.75) (layer "B.Cu") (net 1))
 (segment (start 144.713827 78.22) (end 130.66 78.22) (width 0.75) (layer "B.Cu") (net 2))
 (segment (start 130.67 86.44) (end 132.47 84.64) (width 0.75) (layer "B.Cu") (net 2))
 (segment (start 128.17 80.71) (end 128.17 85.51) (width 0.75) (layer "B.Cu") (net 2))
 (segment (start 146.553572 81.443572) (end 146.553572 80.059745) (width 0.75) (layer "B.Cu") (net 2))
 (segment (start 152.615714 82.33) (end 147.44 82.33) (width 0.75) (layer "B.Cu") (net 2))
 (segment (start 129.1 86.44) (end 130.67 86.44) (width 0.75) (layer "B.Cu") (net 2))
 (segment (start 130.66 78.22) (end 128.17 80.71) (width 0.75) (layer "B.Cu") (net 2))
 (segment (start 146.553572 80.059745) (end 144.713827 78.22) (width 0.75) (layer "B.Cu") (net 2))
 (segment (start 128.17 85.51) (end 129.1 86.44) (width 0.75) (layer "B.Cu") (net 2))
 (segment (start 147.44 82.33) (end 146.553572 81.443572) (width 0.75) (layer "B.Cu") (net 2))
 (segment (start 154.295714 80.65) (end 152.615714 82.33) (width 0.75) (layer "B.Cu") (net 2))
 (segment (start 137.93 86.94) (end 143.583502 86.94) (width 0.7) (layer "B.Cu") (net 4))
 (segment (start 145.128572 85.39493) (end 145.128572 80.65) (width 0.7) (layer "B.Cu") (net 4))
 (segment (start 137.55 86.56) (end 137.93 86.94) (width 0.7) (layer "B.Cu") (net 4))
 (segment (start 143.583502 86.94) (end 145.128572 85.39493) (width 0.7) (layer "B.Cu") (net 4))
 (segment (start 137.55 84.64) (end 137.55 86.56) (width 0.7) (layer "B.Cu") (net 4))
 (segment (start 151.24 79.49) (end 151.77 78.96) (width 0.7) (layer "B.Cu") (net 7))
 (segment (start 138.43 74.45) (end 137.61 73.63) (width 0.7) (layer "B.Cu") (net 7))
 (segment (start 151.24 80.65) (end 151.24 79.49) (width 0.7) (layer "B.Cu") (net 7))
 (segment (start 158.84 81.47) (end 158.84 77.3) (width 0.7) (layer "B.Cu") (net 7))
 (segment (start 151.77 78.96) (end 154.97 78.96) (width 0.7) (layer "B.Cu") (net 7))
 (segment (start 158.84 77.3) (end 155.99 74.45) (width 0.7) (layer "B.Cu") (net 7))
 (segment (start 142.24 69.4) (end 142.63 69.4) (width 0.7) (layer "B.Cu") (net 7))
 (segment (start 155.71 81.32) (end 156.44 82.05) (width 0.7) (layer "B.Cu") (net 7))
 (segment (start 137.61 73.63) (end 137.61 71.92) (width 0.7) (layer "B.Cu") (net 7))
 (segment (start 158.26 82.05) (end 158.84 81.47) (width 0.7) (layer "B.Cu") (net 7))
 (segment (start 156.44 82.05) (end 158.26 82.05) (width 0.7) (layer "B.Cu") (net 7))
 (segment (start 140.41 71.23) (end 142.24 69.4) (width 0.7) (layer "B.Cu") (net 7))
 (segment (start 154.97 78.96) (end 155.71 79.7) (width 0.7) (layer "B.Cu") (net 7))
 (segment (start 137.61 71.92) (end 138.3 71.23) (width 0.7) (layer "B.Cu") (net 7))
 (segment (start 155.99 74.45) (end 138.43 74.45) (width 0.7) (layer "B.Cu") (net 7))
 (segment (start 155.71 79.7) (end 155.71 81.32) (width 0.7) (layer "B.Cu") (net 7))
 (segment (start 138.3 71.23) (end 140.41 71.23) (width 0.7) (layer "B.Cu") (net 7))
 (segment (start 146.445 76.425) (end 134.765 76.425) (width 0.75) (layer "B.Cu") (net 11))
 (segment (start 132.47 74.13) (end 132.47 69.4) (width 0.75) (layer "B.Cu") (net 11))
 (segment (start 148.184286 78.164286) (end 146.445 76.425) (width 0.75) (layer "B.Cu") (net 11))
 (segment (start 148.184286 80.65) (end 148.184286 78.164286) (width 0.75) (layer "B.Cu") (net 11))
 (segment (start 134.765 76.425) (end 132.47 74.13) (width 0.75) (layer "B.Cu") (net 11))
 (segment (start 148.31 67.6) (end 142.88 73.03) (width 0.75) (layer "B.Cu") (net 19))
 (segment (start 148.31 65) (end 148.31 67.6) (width 0.75) (layer "B.Cu") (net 19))
 (segment (start 142.88 73.03) (end 142.072858 73.03) (width 0.75) (layer "B.Cu") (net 19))
 (segment (start 157.351428 73.03) (end 157.351428 61.931428) (width 0.75) (layer "B.Cu") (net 20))
 (segment (start 157.351428 61.931428) (end 155.405 59.985) (width 0.75) (layer "B.Cu") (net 20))
 (segment (start 155.405 59.985) (end 150.785 59.985) (width 0.75) (layer "B.Cu") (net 20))
 (segment (start 150.785 59.985) (end 148.31 62.46) (width 0.75) (layer "B.Cu") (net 20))
 (segment (start 150.85 65) (end 150.85 67.308572) (width 0.75) (layer "B.Cu") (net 21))
 (segment (start 150.85 67.308572) (end 145.128572 73.03) (width 0.75) (layer "B.Cu") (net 21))
 (segment (start 156.06 62.65) (end 154.395 60.985) (width 0.75) (layer "B.Cu") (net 22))
 (segment (start 152.325 60.985) (end 150.85 62.46) (width 0.75) (layer "B.Cu") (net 22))
 (segment (start 154.295714 73.03) (end 156.06 71.265714) (width 0.75) (layer "B.Cu") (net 22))
 (segment (start 156.06 71.265714) (end 156.06 62.65) (width 0.75) (layer "B.Cu") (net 22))
 (segment (start 154.395 60.985) (end 152.325 60.985) (width 0.75) (layer "B.Cu") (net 22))
 (segment (start 153.39 67.824286) (end 153.39 65) (width 0.75) (layer "B.Cu") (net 23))
 (segment (start 148.184286 73.03) (end 153.39 67.824286) (width 0.75) (layer "B.Cu") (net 23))
 (segment (start 154.86 68.93) (end 154.865 68.925) (width 0.75) (layer "B.Cu") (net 24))
 (segment (start 151.24 73.03) (end 154.86 69.41) (width 0.75) (layer "B.Cu") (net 24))
 (segment (start 154.865 63.935) (end 153.39 62.46) (width 0.75) (layer "B.Cu") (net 24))
 (segment (start 154.86 69.41) (end 154.86 68.93) (width 0.75) (layer "B.Cu") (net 24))
 (segment (start 154.865 68.925) (end 154.865 63.935) (width 0.75) (layer "B.Cu") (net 24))
 (segment (start 130.16 65) (end 130.16 69.17) (width 0.75) (layer "B.Cu") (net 12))
 (segment (start 130.16 69.17) (end 129.93 69.4) (width 0.75) (layer "B.Cu") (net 12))
 (segment (start 131.77 82.44) (end 126.53 82.44) (width 0.75) (layer "F.Cu") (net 6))
 (via (at 126.53 82.44) (size 1) (drill 0.5) (layers "F.Cu" "B.Cu") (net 6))
 (via (at 131.77 82.44) (size 1) (drill 0.5) (layers "F.Cu" "B.Cu") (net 6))
 (segment (start 119.22 60.31) (end 128.01 60.31) (width 0.75) (layer "B.Cu") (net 6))
 (segment (start 141.115 83.125) (end 138.645 83.125) (width 0.75) (layer "B.Cu") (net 6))
 (segment (start 142.63 84.64) (end 141.115 83.125) (width 0.75) (layer "B.Cu") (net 6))
 (segment (start 117.87 74.48) (end 117.87 61.66) (width 0.75) (layer "B.Cu") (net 6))
 (segment (start 138.645 83.125) (end 137.96 82.44) (width 0.75) (layer "B.Cu") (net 6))
 (segment (start 117.87 61.66) (end 119.22 60.31) (width 0.75) (layer "B.Cu") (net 6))
 (segment (start 125.83 82.44) (end 117.87 74.48) (width 0.75) (layer "B.Cu") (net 6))
 (segment (start 137.96 82.44) (end 131.77 82.44) (width 0.75) (layer "B.Cu") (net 6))
 (segment (start 126.53 82.44) (end 125.83 82.44) (width 0.75) (layer "B.Cu") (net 6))
 (segment (start 128.01 60.31) (end 130.16 62.46) (width 0.75) (layer "B.Cu") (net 6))
 (segment (start 137.55 67.93) (end 137.55 69.4) (width 0.75) (layer "B.Cu") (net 9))
 (segment (start 134.62 65) (end 137.55 67.93) (width 0.75) (layer "B.Cu") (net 9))
 (segment (start 132.7 65) (end 134.62 65) (width 0.75) (layer "B.Cu") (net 9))
 (segment (start 134.76 62.46) (end 140.09 67.79) (width 0.75) (layer "B.Cu") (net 8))
 (segment (start 132.7 62.46) (end 134.76 62.46) (width 0.75) (layer "B.Cu") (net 8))
 (segment (start 140.09 67.79) (end 140.09 69.4) (width 0.75) (layer "B.Cu") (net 8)))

